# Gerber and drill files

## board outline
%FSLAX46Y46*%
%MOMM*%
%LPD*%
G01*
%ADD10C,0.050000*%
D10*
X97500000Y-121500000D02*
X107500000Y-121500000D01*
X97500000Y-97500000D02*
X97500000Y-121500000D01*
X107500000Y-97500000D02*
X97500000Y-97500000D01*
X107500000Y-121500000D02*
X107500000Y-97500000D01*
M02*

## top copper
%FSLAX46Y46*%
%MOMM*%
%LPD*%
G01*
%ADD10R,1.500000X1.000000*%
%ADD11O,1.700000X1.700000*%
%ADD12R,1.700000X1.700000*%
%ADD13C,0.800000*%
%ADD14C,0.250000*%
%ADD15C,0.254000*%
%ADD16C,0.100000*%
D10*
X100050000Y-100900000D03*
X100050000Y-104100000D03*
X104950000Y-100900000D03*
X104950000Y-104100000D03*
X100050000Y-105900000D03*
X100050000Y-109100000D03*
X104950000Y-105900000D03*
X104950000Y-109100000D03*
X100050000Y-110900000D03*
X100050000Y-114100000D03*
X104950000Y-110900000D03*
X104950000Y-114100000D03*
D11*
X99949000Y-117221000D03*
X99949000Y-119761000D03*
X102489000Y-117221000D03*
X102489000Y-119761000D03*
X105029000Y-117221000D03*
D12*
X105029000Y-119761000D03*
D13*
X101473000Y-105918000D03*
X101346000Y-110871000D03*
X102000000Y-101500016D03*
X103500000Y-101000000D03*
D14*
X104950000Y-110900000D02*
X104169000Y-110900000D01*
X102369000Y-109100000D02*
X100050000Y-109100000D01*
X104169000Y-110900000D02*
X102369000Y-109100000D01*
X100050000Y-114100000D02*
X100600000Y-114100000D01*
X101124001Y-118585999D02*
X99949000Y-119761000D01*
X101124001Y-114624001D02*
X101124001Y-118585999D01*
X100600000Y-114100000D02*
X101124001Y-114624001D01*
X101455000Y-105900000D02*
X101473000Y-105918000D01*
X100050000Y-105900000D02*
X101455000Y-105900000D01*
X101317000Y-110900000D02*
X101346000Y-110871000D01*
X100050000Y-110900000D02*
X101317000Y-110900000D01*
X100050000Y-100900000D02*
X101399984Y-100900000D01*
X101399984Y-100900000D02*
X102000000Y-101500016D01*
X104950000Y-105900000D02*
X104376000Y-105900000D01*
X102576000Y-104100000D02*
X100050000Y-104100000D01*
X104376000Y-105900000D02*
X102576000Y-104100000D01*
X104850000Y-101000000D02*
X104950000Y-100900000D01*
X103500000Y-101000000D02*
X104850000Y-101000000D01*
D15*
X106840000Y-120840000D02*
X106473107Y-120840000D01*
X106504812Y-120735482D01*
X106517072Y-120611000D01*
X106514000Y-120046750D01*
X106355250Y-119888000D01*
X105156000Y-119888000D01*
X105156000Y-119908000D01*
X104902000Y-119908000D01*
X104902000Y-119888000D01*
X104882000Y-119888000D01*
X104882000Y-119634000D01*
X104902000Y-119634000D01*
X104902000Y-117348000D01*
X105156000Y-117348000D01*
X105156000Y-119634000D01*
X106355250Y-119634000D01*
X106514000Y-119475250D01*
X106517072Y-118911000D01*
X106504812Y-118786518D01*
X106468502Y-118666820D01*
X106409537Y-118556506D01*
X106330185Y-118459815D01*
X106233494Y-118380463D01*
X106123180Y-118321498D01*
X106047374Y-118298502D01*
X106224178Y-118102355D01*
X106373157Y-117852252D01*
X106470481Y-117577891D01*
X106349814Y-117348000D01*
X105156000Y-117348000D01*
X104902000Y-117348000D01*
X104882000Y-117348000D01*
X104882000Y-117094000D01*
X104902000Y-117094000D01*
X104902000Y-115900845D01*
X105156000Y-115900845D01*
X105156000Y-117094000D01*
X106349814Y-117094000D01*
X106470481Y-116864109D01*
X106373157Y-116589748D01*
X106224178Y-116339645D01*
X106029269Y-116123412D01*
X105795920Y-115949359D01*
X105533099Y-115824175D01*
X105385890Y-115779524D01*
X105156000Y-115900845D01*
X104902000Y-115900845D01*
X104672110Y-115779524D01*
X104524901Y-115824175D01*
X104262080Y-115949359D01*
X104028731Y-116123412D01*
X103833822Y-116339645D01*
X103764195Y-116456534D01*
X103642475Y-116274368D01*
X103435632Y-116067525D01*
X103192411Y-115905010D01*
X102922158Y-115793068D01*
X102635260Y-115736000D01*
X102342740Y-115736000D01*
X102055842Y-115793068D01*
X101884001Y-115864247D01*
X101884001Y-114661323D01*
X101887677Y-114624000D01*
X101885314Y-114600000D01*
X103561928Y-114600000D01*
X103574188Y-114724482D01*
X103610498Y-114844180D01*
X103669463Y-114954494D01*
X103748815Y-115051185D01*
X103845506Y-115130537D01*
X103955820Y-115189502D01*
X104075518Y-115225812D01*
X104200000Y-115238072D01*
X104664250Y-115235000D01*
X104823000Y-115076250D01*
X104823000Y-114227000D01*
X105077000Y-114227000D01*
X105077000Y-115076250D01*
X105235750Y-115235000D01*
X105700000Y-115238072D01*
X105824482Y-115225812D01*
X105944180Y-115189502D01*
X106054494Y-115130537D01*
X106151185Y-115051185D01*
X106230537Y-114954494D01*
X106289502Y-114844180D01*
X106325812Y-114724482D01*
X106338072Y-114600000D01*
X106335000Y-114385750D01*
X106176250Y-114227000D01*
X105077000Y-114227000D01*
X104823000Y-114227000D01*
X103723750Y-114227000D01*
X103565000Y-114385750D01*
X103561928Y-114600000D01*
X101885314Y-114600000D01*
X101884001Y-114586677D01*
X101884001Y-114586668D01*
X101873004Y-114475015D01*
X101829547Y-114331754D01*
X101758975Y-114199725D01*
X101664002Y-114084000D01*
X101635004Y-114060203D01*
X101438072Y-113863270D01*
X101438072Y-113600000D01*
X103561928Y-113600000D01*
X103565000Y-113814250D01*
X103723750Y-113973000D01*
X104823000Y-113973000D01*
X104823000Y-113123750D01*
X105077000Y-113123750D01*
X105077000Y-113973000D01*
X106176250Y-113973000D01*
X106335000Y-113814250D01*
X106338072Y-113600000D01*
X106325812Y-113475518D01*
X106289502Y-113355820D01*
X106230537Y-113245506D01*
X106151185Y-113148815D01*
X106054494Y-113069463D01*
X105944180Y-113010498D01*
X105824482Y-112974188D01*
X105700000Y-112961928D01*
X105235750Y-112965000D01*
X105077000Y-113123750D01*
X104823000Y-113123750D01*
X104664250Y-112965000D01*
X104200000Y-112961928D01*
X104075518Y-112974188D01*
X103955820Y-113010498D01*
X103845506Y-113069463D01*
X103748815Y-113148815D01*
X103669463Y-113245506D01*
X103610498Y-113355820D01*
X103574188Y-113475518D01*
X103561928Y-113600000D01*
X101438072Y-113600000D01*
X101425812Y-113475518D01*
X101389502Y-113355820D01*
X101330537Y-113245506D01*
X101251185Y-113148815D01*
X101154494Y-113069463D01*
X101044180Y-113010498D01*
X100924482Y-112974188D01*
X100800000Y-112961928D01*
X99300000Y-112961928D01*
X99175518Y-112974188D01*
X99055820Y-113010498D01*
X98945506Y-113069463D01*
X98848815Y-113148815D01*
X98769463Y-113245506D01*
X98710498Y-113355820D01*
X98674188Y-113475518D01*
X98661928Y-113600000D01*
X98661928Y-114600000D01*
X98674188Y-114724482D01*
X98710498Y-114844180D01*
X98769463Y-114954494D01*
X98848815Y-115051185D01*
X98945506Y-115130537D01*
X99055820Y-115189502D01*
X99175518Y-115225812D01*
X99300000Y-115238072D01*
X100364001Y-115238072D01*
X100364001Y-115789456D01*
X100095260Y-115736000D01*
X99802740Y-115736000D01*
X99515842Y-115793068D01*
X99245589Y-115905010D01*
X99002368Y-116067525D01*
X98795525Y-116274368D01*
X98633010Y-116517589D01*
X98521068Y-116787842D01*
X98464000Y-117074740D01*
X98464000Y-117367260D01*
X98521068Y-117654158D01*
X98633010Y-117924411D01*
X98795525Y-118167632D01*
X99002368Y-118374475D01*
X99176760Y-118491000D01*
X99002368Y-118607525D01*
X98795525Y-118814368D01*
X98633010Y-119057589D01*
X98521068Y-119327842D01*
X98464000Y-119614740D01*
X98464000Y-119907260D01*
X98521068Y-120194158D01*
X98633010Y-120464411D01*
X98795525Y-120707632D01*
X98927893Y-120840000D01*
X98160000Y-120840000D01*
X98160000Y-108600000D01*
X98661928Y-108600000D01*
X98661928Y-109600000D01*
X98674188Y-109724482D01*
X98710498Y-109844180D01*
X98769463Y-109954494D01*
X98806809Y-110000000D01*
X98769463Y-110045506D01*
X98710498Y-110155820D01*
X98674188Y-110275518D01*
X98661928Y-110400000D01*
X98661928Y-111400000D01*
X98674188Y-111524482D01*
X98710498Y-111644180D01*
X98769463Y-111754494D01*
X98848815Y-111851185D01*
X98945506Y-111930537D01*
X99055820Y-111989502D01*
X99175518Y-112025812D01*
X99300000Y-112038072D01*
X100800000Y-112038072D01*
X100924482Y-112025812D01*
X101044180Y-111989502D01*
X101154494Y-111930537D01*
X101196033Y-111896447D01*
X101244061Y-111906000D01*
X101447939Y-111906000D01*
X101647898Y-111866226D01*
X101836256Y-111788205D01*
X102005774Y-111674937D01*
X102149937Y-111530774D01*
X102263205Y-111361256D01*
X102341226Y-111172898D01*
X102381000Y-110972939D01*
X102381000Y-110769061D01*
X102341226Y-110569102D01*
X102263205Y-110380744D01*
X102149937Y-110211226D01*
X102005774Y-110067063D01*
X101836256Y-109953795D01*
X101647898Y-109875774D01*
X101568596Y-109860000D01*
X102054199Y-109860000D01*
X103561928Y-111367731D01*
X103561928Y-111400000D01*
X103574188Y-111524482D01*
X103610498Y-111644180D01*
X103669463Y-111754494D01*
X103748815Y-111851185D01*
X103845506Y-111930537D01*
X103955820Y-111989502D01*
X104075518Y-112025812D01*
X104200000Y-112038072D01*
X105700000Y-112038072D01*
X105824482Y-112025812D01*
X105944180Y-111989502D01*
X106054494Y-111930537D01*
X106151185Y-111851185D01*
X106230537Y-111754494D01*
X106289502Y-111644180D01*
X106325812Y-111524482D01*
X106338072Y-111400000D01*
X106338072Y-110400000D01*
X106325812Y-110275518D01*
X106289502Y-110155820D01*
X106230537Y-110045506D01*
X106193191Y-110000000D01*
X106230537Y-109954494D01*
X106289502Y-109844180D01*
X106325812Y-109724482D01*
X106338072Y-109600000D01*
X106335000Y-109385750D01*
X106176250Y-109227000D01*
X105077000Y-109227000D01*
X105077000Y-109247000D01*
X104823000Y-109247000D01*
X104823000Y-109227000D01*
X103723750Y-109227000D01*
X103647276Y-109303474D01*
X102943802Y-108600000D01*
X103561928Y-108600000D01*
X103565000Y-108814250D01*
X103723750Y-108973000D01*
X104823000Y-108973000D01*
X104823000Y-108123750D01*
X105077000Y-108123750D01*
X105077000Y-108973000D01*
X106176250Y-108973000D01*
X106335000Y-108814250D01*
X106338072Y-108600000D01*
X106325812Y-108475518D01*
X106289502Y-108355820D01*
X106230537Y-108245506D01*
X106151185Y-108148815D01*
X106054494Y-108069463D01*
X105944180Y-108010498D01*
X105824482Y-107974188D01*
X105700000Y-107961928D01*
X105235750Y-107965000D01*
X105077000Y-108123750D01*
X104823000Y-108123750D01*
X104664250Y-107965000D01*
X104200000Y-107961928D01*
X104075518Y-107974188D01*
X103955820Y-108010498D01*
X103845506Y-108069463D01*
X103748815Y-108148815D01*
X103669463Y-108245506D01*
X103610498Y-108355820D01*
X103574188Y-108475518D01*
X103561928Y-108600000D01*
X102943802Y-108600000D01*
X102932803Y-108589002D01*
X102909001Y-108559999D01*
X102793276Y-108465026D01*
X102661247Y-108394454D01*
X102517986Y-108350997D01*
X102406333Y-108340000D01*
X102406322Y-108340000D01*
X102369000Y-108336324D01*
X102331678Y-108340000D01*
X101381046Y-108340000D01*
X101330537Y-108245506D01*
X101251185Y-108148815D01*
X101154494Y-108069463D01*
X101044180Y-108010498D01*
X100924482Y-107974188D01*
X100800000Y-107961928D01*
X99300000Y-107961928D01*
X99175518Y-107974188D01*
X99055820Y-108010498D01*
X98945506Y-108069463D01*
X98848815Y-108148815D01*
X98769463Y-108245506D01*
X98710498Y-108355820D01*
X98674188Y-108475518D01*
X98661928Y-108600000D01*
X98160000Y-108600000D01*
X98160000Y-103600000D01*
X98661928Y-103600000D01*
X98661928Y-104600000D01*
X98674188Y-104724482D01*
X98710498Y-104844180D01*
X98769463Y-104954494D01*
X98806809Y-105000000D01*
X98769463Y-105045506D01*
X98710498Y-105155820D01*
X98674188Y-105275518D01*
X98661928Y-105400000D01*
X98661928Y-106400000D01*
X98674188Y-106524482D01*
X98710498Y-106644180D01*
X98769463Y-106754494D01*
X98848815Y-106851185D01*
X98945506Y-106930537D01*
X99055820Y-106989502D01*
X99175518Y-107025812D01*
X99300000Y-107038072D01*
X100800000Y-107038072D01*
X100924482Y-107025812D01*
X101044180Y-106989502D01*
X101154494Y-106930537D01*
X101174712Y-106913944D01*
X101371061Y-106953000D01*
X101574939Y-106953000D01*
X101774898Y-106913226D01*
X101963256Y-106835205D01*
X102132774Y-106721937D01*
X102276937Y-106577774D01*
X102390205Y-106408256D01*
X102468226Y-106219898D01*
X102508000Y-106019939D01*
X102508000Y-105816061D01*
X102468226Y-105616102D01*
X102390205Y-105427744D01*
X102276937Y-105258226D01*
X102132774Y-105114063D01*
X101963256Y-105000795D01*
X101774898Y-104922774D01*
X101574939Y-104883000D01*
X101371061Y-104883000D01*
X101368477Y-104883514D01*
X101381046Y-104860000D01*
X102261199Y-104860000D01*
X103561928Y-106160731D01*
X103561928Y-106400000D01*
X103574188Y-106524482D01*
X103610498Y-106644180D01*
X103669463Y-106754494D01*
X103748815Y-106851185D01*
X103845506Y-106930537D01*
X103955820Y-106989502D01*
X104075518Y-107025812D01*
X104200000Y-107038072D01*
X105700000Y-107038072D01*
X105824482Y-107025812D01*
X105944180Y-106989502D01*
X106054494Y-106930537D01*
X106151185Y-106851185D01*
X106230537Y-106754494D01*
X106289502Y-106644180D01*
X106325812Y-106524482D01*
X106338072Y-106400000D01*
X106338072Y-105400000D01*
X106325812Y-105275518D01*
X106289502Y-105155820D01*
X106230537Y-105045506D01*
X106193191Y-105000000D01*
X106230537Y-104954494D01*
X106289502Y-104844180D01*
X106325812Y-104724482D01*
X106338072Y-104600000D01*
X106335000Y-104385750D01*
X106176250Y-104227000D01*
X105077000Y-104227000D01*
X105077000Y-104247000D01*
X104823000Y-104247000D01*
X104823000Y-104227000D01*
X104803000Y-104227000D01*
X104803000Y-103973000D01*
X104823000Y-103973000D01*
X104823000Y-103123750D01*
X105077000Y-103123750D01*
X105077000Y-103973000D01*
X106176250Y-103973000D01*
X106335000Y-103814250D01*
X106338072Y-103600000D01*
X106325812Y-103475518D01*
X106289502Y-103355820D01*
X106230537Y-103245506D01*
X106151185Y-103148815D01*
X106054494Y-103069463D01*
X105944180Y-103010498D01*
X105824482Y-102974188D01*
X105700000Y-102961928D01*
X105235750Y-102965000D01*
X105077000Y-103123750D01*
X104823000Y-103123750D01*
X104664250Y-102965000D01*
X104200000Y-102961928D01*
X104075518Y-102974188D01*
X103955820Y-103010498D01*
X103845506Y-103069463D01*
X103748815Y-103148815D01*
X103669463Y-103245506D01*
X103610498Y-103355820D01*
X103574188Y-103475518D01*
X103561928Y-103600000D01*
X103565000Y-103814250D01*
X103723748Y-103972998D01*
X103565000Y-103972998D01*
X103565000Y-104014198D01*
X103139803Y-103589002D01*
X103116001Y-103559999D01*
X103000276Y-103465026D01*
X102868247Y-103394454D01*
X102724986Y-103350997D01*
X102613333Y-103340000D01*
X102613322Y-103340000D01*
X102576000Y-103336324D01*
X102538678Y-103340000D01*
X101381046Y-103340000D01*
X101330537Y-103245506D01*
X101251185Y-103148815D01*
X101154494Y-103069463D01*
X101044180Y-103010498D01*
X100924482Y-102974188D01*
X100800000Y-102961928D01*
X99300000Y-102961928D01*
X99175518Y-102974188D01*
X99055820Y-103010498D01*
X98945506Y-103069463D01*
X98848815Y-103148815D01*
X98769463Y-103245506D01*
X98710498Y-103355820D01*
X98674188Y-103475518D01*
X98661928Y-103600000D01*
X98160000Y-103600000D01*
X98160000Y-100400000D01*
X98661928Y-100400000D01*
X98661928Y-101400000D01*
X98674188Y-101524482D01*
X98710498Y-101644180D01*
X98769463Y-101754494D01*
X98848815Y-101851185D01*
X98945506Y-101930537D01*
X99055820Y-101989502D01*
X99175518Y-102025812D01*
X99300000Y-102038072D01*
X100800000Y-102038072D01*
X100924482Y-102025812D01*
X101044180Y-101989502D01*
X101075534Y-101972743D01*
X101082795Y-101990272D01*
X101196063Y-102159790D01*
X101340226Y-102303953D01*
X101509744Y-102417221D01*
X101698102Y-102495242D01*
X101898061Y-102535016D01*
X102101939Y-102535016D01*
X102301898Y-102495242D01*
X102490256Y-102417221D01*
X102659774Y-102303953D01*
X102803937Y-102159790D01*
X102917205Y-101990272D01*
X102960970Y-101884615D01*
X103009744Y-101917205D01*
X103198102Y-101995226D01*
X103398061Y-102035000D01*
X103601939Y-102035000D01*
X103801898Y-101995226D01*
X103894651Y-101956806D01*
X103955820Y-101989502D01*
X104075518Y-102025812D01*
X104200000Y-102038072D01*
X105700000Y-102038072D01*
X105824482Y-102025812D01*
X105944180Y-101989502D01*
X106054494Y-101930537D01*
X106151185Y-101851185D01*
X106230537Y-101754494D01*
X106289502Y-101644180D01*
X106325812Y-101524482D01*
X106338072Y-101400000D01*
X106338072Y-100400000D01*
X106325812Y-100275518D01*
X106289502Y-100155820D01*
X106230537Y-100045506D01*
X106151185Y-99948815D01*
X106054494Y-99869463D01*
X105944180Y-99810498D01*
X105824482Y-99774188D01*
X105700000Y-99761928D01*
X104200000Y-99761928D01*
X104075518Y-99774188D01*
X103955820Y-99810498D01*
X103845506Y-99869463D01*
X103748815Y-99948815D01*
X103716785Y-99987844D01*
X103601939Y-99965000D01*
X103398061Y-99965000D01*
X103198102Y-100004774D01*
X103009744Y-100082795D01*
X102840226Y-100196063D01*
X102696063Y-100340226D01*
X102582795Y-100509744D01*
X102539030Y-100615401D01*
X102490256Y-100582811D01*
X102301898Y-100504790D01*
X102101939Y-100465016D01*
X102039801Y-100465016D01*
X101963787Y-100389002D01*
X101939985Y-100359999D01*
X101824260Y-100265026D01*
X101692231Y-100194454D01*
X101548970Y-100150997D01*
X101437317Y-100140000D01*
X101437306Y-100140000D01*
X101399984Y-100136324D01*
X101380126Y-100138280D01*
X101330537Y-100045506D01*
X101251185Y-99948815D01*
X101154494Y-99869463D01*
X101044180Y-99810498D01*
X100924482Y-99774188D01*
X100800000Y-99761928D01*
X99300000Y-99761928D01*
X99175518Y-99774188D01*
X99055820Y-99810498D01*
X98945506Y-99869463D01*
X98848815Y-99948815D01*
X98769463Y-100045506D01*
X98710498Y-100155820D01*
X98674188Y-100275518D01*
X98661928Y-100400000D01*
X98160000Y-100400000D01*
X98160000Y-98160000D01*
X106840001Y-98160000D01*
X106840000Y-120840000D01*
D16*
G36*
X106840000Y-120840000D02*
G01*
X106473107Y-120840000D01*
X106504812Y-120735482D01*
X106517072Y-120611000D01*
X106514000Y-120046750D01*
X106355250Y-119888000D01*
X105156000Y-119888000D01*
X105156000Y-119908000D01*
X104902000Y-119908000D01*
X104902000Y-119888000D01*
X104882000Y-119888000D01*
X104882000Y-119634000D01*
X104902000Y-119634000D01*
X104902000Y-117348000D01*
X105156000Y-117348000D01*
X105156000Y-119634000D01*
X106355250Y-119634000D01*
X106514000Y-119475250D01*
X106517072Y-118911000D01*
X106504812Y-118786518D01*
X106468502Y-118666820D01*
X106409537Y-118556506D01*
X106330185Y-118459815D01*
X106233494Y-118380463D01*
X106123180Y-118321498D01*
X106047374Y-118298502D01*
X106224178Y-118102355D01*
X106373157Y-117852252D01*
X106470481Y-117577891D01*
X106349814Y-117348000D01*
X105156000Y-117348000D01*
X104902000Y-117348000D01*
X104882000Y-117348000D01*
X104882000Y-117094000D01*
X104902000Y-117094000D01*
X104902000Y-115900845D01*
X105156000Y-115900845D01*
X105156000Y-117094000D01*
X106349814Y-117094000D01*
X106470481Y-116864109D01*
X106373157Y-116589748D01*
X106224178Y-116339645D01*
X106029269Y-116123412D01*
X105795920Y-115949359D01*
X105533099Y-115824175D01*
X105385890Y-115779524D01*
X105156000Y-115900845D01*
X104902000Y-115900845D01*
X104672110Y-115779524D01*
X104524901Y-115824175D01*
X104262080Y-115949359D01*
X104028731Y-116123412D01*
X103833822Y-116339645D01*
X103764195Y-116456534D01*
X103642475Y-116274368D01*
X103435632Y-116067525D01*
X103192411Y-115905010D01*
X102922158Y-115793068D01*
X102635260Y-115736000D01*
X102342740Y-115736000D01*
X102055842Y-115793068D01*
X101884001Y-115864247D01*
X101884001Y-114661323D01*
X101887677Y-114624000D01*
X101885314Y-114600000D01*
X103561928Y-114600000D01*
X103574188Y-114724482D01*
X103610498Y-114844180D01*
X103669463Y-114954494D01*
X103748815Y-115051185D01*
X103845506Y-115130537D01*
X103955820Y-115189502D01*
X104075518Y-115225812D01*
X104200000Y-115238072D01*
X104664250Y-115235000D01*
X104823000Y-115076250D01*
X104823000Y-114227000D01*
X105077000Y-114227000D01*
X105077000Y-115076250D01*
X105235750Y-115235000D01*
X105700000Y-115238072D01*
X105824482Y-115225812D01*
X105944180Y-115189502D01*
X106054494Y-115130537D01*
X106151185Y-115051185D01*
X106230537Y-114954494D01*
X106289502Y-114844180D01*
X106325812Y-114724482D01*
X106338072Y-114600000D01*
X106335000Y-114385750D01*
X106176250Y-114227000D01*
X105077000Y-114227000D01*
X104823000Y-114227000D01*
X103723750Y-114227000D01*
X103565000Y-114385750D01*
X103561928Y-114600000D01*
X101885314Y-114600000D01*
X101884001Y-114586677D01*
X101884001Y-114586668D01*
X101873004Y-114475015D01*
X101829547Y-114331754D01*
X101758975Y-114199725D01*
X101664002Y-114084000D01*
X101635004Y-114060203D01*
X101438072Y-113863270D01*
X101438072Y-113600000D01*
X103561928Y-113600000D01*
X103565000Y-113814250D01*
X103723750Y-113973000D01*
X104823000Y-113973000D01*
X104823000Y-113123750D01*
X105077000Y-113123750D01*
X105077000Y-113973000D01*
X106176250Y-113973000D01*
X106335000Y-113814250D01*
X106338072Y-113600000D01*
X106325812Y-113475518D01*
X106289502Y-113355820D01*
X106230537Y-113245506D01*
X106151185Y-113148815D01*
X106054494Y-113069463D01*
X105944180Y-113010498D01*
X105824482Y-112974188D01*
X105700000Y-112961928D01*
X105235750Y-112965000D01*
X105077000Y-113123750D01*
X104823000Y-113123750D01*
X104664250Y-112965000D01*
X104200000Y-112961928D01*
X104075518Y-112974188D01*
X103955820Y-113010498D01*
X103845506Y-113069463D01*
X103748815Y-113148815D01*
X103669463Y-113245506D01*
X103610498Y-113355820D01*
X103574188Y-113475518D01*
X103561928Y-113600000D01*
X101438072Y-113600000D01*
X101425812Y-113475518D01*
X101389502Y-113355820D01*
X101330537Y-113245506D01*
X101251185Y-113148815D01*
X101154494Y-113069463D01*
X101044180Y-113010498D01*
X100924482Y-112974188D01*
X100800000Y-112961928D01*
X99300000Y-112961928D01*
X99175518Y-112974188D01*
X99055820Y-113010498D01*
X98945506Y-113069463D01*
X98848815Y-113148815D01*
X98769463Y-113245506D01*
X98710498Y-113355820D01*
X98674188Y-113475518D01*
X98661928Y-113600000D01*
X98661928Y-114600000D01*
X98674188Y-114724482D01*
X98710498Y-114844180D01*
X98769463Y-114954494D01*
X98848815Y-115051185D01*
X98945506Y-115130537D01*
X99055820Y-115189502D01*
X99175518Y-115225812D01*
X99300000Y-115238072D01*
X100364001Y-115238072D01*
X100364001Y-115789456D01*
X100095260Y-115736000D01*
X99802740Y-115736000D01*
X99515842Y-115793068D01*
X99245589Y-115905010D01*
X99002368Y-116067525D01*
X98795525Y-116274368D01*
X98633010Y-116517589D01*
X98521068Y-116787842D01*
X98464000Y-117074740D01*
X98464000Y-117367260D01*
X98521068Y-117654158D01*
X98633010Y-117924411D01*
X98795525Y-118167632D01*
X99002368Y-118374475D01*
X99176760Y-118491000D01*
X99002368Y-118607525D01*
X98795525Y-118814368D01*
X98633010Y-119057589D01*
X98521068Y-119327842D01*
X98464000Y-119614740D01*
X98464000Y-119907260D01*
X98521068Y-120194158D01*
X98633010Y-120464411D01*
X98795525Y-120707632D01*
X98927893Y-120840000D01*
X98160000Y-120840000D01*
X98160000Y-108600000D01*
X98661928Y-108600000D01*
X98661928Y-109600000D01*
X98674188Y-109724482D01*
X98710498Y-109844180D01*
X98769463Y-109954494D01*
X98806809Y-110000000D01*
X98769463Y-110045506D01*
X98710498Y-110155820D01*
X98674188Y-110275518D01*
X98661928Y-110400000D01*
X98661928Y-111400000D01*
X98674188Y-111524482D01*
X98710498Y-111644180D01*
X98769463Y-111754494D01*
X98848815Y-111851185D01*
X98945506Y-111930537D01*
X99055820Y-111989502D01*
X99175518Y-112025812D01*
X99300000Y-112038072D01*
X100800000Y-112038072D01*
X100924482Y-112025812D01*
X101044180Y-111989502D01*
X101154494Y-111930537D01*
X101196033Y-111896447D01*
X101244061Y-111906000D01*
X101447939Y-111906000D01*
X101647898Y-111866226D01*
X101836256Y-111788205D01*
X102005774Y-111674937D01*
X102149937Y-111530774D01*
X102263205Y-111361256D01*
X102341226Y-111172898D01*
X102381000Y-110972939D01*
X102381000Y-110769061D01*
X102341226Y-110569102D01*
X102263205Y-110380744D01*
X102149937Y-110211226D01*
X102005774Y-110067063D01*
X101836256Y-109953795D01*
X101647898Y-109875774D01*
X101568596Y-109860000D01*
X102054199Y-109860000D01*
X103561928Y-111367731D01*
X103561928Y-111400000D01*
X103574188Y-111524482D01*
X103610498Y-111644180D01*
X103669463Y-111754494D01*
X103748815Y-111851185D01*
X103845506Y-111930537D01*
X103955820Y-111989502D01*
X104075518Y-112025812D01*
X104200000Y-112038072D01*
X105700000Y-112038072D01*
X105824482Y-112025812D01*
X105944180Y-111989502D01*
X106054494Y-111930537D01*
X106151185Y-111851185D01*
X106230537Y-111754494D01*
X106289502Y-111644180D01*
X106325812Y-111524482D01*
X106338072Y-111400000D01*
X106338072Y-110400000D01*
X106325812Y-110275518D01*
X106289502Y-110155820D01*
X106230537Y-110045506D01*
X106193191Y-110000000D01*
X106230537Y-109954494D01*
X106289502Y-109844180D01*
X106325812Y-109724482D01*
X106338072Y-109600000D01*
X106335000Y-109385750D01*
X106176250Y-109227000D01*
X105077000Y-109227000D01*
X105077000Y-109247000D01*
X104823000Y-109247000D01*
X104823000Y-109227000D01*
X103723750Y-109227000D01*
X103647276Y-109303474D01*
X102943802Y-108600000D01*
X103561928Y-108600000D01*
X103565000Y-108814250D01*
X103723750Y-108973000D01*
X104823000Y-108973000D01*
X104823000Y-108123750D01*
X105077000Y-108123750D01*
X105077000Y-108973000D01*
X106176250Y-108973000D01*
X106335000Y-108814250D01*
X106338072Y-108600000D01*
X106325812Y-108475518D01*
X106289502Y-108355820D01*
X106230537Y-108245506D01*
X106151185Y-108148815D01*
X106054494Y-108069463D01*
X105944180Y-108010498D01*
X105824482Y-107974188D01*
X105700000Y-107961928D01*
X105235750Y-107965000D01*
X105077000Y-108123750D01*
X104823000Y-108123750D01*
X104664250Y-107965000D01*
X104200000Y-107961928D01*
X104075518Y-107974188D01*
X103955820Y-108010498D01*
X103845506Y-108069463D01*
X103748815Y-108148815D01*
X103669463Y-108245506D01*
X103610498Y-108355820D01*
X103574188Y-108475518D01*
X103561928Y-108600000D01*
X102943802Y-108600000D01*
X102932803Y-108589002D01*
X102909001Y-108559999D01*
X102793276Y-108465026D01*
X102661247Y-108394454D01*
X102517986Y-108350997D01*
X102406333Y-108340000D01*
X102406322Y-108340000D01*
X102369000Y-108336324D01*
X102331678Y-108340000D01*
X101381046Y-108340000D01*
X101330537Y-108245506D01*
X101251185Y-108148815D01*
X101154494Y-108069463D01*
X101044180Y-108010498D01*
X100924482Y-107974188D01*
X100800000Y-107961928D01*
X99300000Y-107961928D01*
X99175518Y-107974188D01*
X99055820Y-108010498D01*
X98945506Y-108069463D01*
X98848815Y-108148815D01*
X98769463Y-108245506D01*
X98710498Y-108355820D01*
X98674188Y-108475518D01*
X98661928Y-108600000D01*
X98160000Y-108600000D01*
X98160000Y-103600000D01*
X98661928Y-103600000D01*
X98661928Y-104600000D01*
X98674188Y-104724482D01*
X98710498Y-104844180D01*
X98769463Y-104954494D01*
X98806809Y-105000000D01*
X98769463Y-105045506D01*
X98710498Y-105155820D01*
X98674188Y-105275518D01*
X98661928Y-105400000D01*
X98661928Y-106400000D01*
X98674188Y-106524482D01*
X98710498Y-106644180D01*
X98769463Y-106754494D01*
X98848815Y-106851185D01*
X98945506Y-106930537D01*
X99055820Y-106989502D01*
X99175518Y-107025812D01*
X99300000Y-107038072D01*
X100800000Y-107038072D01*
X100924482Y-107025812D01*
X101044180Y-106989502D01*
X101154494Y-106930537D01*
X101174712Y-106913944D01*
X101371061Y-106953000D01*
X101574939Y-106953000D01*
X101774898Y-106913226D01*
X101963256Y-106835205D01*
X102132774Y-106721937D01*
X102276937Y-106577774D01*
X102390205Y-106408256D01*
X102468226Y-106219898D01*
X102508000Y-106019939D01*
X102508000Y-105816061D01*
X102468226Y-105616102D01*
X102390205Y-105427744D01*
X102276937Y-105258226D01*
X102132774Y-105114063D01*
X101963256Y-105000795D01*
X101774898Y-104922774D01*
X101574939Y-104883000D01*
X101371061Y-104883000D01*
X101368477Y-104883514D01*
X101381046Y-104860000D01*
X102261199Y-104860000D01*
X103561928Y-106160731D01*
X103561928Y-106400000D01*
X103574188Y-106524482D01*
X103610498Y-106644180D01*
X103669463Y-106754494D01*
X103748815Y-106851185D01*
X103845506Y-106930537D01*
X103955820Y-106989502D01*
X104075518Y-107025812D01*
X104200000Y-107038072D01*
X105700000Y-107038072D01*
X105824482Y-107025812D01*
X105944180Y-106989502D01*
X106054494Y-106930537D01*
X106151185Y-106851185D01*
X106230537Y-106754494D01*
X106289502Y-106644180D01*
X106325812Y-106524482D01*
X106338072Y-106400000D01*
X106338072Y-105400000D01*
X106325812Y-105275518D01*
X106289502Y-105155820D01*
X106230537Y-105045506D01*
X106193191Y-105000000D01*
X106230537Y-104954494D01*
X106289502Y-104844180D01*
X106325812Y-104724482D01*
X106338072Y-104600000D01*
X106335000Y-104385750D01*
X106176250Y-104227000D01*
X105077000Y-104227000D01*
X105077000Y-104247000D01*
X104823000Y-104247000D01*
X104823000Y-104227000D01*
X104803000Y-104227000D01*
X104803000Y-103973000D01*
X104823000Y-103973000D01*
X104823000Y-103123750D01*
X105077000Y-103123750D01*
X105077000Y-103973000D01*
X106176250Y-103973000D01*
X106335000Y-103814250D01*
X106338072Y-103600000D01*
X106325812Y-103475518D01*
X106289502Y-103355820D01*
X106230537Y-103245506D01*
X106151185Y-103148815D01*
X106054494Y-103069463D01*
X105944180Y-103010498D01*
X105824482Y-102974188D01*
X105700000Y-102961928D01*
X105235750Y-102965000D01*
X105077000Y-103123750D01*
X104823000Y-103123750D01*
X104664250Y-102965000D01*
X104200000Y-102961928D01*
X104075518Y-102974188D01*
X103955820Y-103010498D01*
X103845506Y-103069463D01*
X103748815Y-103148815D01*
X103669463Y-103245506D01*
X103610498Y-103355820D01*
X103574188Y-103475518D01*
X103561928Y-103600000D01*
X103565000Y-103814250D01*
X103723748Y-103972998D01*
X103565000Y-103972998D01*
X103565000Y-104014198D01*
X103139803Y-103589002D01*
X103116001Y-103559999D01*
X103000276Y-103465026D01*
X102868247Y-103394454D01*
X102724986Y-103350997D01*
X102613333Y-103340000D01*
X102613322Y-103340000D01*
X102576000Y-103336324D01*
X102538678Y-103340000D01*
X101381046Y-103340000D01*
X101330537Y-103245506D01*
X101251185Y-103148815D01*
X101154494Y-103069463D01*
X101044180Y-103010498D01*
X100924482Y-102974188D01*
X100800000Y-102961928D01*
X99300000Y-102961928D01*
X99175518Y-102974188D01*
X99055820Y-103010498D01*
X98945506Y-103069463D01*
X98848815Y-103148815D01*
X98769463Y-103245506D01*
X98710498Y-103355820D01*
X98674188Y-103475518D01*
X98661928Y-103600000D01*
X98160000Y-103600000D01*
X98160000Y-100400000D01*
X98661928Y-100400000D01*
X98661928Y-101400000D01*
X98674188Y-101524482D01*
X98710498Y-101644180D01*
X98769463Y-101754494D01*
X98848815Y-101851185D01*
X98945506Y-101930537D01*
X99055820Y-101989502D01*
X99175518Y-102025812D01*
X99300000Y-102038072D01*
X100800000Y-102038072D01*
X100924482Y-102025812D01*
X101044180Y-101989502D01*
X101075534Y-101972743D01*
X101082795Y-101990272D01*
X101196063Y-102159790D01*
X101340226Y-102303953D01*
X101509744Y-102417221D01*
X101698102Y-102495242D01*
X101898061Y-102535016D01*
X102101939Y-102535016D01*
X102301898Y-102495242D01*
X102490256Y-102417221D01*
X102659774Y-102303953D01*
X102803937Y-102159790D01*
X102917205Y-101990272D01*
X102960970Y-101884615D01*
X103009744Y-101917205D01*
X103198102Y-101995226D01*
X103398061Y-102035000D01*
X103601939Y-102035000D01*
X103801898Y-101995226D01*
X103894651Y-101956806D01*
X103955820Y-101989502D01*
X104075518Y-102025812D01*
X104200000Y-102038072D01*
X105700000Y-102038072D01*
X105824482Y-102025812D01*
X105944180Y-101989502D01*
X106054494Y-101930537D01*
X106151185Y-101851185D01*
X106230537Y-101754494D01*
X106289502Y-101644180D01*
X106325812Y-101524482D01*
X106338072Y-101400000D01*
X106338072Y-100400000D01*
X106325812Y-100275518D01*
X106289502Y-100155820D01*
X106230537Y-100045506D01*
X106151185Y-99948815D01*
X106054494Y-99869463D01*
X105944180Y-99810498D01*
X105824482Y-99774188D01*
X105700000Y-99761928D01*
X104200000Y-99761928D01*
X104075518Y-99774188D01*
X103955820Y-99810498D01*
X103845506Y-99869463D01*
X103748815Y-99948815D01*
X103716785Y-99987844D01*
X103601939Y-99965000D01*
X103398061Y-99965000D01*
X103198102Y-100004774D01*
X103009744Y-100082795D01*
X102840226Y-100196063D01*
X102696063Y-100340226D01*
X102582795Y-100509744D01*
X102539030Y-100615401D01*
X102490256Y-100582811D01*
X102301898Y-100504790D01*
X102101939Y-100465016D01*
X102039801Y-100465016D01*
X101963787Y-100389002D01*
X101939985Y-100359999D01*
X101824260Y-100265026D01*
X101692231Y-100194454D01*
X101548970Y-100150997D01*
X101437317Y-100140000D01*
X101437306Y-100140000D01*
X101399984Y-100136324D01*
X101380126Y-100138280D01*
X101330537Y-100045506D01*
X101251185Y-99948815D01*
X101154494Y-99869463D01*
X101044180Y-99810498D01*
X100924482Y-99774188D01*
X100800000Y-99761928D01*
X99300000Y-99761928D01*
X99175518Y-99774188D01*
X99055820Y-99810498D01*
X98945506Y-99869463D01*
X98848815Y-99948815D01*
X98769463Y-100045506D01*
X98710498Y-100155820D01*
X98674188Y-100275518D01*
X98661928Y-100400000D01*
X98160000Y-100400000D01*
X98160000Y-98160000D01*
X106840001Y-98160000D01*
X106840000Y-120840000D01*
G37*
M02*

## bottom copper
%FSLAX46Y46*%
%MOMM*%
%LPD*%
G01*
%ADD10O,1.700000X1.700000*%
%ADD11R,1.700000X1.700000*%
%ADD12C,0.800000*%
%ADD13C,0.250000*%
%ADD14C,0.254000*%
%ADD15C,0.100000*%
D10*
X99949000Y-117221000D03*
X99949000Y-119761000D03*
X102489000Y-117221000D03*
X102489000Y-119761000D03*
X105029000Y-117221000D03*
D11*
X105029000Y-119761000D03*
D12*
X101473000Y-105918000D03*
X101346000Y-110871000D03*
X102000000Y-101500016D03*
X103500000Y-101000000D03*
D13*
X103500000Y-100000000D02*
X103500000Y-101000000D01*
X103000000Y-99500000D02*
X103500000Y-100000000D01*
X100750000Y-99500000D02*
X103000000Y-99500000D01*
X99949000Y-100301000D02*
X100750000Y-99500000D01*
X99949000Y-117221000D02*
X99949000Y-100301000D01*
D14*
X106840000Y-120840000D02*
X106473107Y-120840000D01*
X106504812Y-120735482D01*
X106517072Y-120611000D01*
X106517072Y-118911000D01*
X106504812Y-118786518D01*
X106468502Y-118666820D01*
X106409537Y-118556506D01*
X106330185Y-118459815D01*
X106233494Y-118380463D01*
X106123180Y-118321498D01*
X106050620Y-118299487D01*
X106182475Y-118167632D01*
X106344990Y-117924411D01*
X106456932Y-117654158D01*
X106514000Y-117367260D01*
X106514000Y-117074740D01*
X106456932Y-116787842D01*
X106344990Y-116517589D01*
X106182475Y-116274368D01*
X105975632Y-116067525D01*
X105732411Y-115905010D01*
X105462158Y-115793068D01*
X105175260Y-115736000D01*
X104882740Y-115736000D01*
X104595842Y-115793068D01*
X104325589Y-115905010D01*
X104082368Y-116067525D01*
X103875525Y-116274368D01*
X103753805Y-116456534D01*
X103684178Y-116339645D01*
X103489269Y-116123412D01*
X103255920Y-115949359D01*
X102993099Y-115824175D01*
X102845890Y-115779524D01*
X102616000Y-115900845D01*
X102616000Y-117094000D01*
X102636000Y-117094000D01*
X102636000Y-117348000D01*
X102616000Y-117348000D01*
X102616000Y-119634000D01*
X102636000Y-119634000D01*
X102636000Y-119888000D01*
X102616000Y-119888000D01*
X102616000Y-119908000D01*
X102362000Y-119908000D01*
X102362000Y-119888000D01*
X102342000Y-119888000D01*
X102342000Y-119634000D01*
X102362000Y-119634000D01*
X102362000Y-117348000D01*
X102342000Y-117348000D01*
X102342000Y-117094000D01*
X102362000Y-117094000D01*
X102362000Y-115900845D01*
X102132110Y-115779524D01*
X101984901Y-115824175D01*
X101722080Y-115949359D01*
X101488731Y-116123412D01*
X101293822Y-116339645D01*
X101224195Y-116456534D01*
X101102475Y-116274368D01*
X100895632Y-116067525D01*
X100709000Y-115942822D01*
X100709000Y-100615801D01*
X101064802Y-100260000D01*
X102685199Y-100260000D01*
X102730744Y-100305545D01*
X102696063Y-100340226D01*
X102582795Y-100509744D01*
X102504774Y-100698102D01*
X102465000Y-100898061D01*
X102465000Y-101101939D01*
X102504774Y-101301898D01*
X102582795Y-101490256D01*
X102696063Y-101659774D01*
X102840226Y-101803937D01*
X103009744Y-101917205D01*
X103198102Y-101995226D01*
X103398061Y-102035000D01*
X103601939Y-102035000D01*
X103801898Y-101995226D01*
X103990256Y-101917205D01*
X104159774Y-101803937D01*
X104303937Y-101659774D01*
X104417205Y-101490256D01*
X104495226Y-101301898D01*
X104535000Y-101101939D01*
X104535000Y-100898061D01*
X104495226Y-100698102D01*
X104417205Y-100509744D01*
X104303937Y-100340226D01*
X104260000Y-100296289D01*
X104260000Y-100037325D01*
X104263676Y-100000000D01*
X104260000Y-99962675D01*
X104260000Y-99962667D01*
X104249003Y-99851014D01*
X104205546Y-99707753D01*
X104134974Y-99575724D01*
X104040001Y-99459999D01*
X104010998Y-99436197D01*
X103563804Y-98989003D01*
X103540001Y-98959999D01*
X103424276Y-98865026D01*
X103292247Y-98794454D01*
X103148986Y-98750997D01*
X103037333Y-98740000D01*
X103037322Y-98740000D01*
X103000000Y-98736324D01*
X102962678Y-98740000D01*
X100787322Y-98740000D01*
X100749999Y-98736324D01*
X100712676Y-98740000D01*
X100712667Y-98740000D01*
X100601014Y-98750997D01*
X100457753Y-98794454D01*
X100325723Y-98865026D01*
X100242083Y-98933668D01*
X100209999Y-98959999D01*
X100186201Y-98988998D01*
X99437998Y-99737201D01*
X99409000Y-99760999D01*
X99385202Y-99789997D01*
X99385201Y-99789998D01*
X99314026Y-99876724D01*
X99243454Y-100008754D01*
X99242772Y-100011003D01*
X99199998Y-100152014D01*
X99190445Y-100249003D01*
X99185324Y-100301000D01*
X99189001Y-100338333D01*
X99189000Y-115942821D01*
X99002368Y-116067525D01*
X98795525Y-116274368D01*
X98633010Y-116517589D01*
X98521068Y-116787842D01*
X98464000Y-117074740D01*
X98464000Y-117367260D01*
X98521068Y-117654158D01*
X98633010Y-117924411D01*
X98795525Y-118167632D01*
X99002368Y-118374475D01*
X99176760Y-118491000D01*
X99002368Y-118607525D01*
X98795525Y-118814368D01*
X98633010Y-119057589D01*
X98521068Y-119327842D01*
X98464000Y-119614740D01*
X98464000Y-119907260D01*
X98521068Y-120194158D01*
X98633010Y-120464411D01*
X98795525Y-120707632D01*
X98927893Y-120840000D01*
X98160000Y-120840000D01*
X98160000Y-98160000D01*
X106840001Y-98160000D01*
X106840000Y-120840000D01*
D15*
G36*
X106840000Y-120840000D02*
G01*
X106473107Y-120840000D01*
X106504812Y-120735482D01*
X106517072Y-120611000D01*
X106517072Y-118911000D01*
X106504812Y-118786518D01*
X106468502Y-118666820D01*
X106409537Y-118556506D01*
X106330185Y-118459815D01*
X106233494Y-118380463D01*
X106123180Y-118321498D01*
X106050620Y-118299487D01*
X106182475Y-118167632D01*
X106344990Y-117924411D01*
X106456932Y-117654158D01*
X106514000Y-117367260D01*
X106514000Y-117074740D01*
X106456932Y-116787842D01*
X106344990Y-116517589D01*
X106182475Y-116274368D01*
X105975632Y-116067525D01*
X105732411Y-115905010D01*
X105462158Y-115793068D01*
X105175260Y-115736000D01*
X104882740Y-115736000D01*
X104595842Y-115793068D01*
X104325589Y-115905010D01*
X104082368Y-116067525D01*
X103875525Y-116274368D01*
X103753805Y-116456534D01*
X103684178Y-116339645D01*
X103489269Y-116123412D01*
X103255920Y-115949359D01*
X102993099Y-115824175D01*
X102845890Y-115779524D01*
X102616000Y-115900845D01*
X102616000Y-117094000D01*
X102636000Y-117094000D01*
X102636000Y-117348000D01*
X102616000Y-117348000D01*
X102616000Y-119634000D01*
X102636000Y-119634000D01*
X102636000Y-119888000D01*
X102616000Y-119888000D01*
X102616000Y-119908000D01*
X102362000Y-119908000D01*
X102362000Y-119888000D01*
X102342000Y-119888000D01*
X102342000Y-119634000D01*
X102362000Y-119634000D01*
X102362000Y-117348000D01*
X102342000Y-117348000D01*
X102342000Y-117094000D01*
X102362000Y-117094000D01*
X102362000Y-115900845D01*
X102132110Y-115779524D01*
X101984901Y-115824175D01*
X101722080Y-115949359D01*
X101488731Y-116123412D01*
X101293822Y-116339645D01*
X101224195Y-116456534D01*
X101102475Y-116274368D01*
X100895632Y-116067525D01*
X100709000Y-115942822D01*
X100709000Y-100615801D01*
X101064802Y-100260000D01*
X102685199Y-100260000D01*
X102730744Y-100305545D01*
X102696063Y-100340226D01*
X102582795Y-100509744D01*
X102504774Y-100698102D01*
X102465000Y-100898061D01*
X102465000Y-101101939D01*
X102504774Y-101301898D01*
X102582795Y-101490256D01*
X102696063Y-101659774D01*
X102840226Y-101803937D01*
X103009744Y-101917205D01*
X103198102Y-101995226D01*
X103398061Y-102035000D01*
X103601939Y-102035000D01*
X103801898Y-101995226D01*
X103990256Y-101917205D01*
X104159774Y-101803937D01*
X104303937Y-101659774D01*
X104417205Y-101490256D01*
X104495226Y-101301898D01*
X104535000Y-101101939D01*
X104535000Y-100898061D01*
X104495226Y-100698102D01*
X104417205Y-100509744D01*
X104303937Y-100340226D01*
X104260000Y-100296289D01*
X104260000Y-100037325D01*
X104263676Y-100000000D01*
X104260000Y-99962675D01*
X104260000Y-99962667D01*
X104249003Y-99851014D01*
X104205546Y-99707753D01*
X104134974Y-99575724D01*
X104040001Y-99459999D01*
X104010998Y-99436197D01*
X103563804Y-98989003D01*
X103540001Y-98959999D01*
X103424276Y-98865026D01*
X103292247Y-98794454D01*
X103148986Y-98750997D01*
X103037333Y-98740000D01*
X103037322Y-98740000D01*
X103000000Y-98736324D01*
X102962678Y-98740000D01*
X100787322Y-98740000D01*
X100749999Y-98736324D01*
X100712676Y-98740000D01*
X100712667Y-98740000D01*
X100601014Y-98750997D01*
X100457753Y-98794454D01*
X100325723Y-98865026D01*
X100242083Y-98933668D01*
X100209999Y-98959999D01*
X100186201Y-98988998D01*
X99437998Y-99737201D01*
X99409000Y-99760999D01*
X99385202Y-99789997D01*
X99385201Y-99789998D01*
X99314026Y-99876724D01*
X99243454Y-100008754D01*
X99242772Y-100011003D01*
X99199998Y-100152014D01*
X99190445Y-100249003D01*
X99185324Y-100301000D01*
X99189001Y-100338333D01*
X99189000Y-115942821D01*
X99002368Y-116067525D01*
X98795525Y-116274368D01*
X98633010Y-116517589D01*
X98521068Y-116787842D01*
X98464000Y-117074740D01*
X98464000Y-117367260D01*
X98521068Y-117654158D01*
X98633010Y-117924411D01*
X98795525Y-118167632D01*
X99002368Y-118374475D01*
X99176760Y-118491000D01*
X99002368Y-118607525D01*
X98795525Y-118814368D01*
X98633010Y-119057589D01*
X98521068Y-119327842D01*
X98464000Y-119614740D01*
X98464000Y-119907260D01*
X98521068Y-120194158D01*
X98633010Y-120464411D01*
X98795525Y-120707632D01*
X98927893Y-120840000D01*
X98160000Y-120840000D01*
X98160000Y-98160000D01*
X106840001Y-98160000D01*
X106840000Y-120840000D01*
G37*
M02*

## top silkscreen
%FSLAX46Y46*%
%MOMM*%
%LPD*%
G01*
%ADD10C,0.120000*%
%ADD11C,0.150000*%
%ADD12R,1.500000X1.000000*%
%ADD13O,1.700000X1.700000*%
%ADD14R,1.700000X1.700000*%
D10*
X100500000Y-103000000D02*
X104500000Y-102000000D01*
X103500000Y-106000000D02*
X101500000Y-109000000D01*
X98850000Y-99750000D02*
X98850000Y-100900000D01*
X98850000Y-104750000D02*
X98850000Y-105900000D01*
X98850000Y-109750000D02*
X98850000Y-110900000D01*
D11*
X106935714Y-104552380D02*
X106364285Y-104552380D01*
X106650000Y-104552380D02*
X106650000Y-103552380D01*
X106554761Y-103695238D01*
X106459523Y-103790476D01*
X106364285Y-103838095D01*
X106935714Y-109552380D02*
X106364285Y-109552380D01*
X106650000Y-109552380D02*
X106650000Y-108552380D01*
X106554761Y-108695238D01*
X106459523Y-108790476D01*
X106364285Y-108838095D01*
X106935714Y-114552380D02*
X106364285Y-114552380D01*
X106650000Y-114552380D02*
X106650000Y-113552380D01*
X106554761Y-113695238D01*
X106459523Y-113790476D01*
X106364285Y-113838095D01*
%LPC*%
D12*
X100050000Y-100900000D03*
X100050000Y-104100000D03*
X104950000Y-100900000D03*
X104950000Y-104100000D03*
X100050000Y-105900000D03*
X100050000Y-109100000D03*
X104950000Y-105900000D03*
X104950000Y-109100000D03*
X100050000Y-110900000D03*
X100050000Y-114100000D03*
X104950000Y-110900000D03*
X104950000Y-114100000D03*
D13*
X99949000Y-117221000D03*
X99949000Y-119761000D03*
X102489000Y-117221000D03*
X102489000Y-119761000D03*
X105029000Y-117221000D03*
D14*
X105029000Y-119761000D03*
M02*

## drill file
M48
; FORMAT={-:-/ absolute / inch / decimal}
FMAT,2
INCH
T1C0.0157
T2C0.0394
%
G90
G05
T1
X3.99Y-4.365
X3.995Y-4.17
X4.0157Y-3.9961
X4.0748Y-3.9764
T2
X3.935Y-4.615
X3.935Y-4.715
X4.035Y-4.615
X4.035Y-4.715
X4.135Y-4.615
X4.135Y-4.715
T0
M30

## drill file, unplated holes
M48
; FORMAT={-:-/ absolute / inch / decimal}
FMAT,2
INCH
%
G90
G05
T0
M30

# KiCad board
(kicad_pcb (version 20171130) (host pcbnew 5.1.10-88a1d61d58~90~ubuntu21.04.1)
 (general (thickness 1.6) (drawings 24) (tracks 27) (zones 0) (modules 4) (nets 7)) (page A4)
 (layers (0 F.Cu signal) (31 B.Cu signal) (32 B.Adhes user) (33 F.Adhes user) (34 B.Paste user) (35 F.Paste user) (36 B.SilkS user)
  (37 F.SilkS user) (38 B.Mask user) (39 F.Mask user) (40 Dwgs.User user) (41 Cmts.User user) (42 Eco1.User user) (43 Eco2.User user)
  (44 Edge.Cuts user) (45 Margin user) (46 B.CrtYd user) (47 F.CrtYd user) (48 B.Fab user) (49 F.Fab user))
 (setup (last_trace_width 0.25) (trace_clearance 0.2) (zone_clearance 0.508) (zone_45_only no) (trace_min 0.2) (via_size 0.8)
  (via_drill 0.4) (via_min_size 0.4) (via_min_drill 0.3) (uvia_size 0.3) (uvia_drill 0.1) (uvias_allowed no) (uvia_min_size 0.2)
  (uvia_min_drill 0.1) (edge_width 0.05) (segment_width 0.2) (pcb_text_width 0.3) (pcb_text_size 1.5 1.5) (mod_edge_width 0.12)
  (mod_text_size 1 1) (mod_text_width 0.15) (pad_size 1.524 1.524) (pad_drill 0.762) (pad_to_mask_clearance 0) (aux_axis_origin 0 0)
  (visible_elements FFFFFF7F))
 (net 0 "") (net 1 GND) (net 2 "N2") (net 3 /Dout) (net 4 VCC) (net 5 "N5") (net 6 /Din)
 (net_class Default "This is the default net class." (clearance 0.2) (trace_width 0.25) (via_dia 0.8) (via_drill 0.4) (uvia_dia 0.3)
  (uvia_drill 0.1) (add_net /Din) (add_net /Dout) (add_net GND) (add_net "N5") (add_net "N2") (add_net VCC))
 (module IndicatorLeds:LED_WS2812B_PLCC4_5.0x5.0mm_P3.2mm (layer F.Cu) (at 102.5 102.5 180)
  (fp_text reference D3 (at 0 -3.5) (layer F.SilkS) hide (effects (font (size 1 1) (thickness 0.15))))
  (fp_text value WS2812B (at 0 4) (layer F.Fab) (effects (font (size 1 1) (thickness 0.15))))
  (fp_line (start 3.65 2.75) (end 3.65 1.6) (layer F.SilkS) (width 0.12))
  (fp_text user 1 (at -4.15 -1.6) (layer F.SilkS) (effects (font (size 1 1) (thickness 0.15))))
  (pad 3 smd rect (at 2.45 1.6 180) (size 1.5 1) (layers F.Cu F.Paste F.Mask) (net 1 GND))
  (pad 4 smd rect (at 2.45 -1.6 180) (size 1.5 1) (layers F.Cu F.Paste F.Mask) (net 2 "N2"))
  (pad 2 smd rect (at -2.45 1.6 180) (size 1.5 1) (layers F.Cu F.Paste F.Mask) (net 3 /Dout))
  (pad 1 smd rect (at -2.45 -1.6 180) (size 1.5 1) (layers F.Cu F.Paste F.Mask) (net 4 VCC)))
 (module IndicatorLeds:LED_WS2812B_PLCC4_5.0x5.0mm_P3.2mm (layer F.Cu) (at 102.5 107.5 180)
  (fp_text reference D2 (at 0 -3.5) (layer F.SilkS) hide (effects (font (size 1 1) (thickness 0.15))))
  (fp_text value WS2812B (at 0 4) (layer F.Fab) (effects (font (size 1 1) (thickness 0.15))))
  (fp_line (start 3.65 2.75) (end 3.65 1.6) (layer F.SilkS) (width 0.12))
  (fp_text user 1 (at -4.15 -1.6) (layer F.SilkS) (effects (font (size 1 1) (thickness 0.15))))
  (pad 3 smd rect (at 2.45 1.6 180) (size 1.5 1) (layers F.Cu F.Paste F.Mask) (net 1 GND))
  (pad 4 smd rect (at 2.45 -1.6 180) (size 1.5 1) (layers F.Cu F.Paste F.Mask) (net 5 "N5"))
  (pad 2 smd rect (at -2.45 1.6 180) (size 1.5 1) (layers F.Cu F.Paste F.Mask) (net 2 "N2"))
  (pad 1 smd rect (at -2.45 -1.6 180) (size 1.5 1) (layers F.Cu F.Paste F.Mask) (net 4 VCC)))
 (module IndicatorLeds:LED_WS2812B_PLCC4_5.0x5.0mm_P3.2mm (layer F.Cu) (at 102.5 112.5 180)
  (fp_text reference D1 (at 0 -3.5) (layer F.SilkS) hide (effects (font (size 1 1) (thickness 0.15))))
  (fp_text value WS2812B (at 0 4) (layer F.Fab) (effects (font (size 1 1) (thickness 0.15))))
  (fp_line (start 3.65 2.75) (end 3.65 1.6) (layer F.SilkS) (width 0.12))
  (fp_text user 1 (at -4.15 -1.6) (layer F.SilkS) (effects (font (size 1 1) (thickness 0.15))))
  (pad 3 smd rect (at 2.45 1.6 180) (size 1.5 1) (layers F.Cu F.Paste F.Mask) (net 1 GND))
  (pad 4 smd rect (at 2.45 -1.6 180) (size 1.5 1) (layers F.Cu F.Paste F.Mask) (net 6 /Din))
  (pad 2 smd rect (at -2.45 1.6 180) (size 1.5 1) (layers F.Cu F.Paste F.Mask) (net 5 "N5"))
  (pad 1 smd rect (at -2.45 -1.6 180) (size 1.5 1) (layers F.Cu F.Paste F.Mask) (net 4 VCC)))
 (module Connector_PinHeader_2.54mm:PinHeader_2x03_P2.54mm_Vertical (layer B.Cu) (at 105.029 119.761 90)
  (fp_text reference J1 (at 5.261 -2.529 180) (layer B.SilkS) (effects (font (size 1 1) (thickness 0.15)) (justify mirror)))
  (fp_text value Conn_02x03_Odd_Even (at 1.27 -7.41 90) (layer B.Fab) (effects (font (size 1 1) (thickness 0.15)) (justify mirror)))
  (pad 6 thru_hole oval (at 2.54 -5.08 90) (size 1.7 1.7) (drill 1) (layers *.Cu *.Mask) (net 3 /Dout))
  (pad 5 thru_hole oval (at 0 -5.08 90) (size 1.7 1.7) (drill 1) (layers *.Cu *.Mask) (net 6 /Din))
  (pad 4 thru_hole oval (at 2.54 -2.54 90) (size 1.7 1.7) (drill 1) (layers *.Cu *.Mask) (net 1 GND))
  (pad 3 thru_hole oval (at 0 -2.54 90) (size 1.7 1.7) (drill 1) (layers *.Cu *.Mask) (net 1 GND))
  (pad 2 thru_hole oval (at 2.54 0 90) (size 1.7 1.7) (drill 1) (layers *.Cu *.Mask) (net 4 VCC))
  (pad 1 thru_hole rect (at 0 0 90) (size 1.7 1.7) (drill 1) (layers *.Cu *.Mask) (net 4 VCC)))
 (gr_line (start 100.5 103) (end 104.5 102) (layer F.SilkS) (width 0.12))
 (gr_line (start 103.5 106) (end 101.5 109) (layer F.SilkS) (width 0.12))
 (gr_line (start 97.5 121.5) (end 107.5 121.5) (layer Edge.Cuts) (width 0.05))
 (gr_line (start 97.5 97.5) (end 97.5 121.5) (layer Edge.Cuts) (width 0.05))
 (gr_line (start 107.5 97.5) (end 97.5 97.5) (layer Edge.Cuts) (width 0.05))
 (gr_line (start 107.5 121.5) (end 107.5 97.5) (layer Edge.Cuts) (width 0.05))
 (segment (start 104.95 110.9) (end 104.169 110.9) (width 0.25) (layer F.Cu) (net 5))
 (segment (start 102.369 109.1) (end 100.05 109.1) (width 0.25) (layer F.Cu) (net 5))
 (segment (start 104.169 110.9) (end 102.369 109.1) (width 0.25) (layer F.Cu) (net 5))
 (segment (start 100.05 114.1) (end 100.6 114.1) (width 0.25) (layer F.Cu) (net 6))
 (segment (start 101.124001 118.585999) (end 99.949 119.761) (width 0.25) (layer F.Cu) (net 6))
 (segment (start 101.124001 114.624001) (end 101.124001 118.585999) (width 0.25) (layer F.Cu) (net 6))
 (segment (start 100.6 114.1) (end 101.124001 114.624001) (width 0.25) (layer F.Cu) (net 6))
 (via (at 101.473 105.918) (size 0.8) (drill 0.4) (layers F.Cu B.Cu) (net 1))
 (segment (start 101.455 105.9) (end 101.473 105.918) (width 0.25) (layer F.Cu) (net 1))
 (segment (start 100.05 105.9) (end 101.455 105.9) (width 0.25) (layer F.Cu) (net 1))
 (via (at 101.346 110.871) (size 0.8) (drill 0.4) (layers F.Cu B.Cu) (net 1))
 (segment (start 101.317 110.9) (end 101.346 110.871) (width 0.25) (layer F.Cu) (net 1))
 (segment (start 100.05 110.9) (end 101.317 110.9) (width 0.25) (layer F.Cu) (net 1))
 (via (at 102 101.500016) (size 0.8) (drill 0.4) (layers F.Cu B.Cu) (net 1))
 (segment (start 100.05 100.9) (end 101.399984 100.9) (width 0.25) (layer F.Cu) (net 1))
 (segment (start 101.399984 100.9) (end 102 101.500016) (width 0.25) (layer F.Cu) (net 1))
 (segment (start 104.95 105.9) (end 104.376 105.9) (width 0.25) (layer F.Cu) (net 2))
 (segment (start 102.576 104.1) (end 100.05 104.1) (width 0.25) (layer F.Cu) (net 2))
 (segment (start 104.376 105.9) (end 102.576 104.1) (width 0.25) (layer F.Cu) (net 2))
 (via (at 103.5 101) (size 0.8) (drill 0.4) (layers F.Cu B.Cu) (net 3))
 (segment (start 104.85 101) (end 104.95 100.9) (width 0.25) (layer F.Cu) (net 3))
 (segment (start 103.5 101) (end 104.85 101) (width 0.25) (layer F.Cu) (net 3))
 (segment (start 103.5 100) (end 103.5 101) (width 0.25) (layer B.Cu) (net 3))
 (segment (start 103 99.5) (end 103.5 100) (width 0.25) (layer B.Cu) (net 3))
 (segment (start 100.75 99.5) (end 103 99.5) (width 0.25) (layer B.Cu) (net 3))
 (segment (start 99.949 100.301) (end 100.75 99.5) (width 0.25) (layer B.Cu) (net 3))
 (segment (start 99.949 117.221) (end 99.949 100.301) (width 0.25) (layer B.Cu) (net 3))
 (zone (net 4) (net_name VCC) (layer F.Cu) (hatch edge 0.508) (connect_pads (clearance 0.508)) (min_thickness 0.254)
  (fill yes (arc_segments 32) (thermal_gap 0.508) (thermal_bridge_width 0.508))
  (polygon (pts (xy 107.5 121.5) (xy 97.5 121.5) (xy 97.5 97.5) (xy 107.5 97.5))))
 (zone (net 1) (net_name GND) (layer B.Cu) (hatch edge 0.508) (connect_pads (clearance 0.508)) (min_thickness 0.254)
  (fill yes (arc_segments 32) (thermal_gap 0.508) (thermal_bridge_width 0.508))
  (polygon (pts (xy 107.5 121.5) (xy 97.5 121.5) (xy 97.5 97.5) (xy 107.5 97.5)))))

